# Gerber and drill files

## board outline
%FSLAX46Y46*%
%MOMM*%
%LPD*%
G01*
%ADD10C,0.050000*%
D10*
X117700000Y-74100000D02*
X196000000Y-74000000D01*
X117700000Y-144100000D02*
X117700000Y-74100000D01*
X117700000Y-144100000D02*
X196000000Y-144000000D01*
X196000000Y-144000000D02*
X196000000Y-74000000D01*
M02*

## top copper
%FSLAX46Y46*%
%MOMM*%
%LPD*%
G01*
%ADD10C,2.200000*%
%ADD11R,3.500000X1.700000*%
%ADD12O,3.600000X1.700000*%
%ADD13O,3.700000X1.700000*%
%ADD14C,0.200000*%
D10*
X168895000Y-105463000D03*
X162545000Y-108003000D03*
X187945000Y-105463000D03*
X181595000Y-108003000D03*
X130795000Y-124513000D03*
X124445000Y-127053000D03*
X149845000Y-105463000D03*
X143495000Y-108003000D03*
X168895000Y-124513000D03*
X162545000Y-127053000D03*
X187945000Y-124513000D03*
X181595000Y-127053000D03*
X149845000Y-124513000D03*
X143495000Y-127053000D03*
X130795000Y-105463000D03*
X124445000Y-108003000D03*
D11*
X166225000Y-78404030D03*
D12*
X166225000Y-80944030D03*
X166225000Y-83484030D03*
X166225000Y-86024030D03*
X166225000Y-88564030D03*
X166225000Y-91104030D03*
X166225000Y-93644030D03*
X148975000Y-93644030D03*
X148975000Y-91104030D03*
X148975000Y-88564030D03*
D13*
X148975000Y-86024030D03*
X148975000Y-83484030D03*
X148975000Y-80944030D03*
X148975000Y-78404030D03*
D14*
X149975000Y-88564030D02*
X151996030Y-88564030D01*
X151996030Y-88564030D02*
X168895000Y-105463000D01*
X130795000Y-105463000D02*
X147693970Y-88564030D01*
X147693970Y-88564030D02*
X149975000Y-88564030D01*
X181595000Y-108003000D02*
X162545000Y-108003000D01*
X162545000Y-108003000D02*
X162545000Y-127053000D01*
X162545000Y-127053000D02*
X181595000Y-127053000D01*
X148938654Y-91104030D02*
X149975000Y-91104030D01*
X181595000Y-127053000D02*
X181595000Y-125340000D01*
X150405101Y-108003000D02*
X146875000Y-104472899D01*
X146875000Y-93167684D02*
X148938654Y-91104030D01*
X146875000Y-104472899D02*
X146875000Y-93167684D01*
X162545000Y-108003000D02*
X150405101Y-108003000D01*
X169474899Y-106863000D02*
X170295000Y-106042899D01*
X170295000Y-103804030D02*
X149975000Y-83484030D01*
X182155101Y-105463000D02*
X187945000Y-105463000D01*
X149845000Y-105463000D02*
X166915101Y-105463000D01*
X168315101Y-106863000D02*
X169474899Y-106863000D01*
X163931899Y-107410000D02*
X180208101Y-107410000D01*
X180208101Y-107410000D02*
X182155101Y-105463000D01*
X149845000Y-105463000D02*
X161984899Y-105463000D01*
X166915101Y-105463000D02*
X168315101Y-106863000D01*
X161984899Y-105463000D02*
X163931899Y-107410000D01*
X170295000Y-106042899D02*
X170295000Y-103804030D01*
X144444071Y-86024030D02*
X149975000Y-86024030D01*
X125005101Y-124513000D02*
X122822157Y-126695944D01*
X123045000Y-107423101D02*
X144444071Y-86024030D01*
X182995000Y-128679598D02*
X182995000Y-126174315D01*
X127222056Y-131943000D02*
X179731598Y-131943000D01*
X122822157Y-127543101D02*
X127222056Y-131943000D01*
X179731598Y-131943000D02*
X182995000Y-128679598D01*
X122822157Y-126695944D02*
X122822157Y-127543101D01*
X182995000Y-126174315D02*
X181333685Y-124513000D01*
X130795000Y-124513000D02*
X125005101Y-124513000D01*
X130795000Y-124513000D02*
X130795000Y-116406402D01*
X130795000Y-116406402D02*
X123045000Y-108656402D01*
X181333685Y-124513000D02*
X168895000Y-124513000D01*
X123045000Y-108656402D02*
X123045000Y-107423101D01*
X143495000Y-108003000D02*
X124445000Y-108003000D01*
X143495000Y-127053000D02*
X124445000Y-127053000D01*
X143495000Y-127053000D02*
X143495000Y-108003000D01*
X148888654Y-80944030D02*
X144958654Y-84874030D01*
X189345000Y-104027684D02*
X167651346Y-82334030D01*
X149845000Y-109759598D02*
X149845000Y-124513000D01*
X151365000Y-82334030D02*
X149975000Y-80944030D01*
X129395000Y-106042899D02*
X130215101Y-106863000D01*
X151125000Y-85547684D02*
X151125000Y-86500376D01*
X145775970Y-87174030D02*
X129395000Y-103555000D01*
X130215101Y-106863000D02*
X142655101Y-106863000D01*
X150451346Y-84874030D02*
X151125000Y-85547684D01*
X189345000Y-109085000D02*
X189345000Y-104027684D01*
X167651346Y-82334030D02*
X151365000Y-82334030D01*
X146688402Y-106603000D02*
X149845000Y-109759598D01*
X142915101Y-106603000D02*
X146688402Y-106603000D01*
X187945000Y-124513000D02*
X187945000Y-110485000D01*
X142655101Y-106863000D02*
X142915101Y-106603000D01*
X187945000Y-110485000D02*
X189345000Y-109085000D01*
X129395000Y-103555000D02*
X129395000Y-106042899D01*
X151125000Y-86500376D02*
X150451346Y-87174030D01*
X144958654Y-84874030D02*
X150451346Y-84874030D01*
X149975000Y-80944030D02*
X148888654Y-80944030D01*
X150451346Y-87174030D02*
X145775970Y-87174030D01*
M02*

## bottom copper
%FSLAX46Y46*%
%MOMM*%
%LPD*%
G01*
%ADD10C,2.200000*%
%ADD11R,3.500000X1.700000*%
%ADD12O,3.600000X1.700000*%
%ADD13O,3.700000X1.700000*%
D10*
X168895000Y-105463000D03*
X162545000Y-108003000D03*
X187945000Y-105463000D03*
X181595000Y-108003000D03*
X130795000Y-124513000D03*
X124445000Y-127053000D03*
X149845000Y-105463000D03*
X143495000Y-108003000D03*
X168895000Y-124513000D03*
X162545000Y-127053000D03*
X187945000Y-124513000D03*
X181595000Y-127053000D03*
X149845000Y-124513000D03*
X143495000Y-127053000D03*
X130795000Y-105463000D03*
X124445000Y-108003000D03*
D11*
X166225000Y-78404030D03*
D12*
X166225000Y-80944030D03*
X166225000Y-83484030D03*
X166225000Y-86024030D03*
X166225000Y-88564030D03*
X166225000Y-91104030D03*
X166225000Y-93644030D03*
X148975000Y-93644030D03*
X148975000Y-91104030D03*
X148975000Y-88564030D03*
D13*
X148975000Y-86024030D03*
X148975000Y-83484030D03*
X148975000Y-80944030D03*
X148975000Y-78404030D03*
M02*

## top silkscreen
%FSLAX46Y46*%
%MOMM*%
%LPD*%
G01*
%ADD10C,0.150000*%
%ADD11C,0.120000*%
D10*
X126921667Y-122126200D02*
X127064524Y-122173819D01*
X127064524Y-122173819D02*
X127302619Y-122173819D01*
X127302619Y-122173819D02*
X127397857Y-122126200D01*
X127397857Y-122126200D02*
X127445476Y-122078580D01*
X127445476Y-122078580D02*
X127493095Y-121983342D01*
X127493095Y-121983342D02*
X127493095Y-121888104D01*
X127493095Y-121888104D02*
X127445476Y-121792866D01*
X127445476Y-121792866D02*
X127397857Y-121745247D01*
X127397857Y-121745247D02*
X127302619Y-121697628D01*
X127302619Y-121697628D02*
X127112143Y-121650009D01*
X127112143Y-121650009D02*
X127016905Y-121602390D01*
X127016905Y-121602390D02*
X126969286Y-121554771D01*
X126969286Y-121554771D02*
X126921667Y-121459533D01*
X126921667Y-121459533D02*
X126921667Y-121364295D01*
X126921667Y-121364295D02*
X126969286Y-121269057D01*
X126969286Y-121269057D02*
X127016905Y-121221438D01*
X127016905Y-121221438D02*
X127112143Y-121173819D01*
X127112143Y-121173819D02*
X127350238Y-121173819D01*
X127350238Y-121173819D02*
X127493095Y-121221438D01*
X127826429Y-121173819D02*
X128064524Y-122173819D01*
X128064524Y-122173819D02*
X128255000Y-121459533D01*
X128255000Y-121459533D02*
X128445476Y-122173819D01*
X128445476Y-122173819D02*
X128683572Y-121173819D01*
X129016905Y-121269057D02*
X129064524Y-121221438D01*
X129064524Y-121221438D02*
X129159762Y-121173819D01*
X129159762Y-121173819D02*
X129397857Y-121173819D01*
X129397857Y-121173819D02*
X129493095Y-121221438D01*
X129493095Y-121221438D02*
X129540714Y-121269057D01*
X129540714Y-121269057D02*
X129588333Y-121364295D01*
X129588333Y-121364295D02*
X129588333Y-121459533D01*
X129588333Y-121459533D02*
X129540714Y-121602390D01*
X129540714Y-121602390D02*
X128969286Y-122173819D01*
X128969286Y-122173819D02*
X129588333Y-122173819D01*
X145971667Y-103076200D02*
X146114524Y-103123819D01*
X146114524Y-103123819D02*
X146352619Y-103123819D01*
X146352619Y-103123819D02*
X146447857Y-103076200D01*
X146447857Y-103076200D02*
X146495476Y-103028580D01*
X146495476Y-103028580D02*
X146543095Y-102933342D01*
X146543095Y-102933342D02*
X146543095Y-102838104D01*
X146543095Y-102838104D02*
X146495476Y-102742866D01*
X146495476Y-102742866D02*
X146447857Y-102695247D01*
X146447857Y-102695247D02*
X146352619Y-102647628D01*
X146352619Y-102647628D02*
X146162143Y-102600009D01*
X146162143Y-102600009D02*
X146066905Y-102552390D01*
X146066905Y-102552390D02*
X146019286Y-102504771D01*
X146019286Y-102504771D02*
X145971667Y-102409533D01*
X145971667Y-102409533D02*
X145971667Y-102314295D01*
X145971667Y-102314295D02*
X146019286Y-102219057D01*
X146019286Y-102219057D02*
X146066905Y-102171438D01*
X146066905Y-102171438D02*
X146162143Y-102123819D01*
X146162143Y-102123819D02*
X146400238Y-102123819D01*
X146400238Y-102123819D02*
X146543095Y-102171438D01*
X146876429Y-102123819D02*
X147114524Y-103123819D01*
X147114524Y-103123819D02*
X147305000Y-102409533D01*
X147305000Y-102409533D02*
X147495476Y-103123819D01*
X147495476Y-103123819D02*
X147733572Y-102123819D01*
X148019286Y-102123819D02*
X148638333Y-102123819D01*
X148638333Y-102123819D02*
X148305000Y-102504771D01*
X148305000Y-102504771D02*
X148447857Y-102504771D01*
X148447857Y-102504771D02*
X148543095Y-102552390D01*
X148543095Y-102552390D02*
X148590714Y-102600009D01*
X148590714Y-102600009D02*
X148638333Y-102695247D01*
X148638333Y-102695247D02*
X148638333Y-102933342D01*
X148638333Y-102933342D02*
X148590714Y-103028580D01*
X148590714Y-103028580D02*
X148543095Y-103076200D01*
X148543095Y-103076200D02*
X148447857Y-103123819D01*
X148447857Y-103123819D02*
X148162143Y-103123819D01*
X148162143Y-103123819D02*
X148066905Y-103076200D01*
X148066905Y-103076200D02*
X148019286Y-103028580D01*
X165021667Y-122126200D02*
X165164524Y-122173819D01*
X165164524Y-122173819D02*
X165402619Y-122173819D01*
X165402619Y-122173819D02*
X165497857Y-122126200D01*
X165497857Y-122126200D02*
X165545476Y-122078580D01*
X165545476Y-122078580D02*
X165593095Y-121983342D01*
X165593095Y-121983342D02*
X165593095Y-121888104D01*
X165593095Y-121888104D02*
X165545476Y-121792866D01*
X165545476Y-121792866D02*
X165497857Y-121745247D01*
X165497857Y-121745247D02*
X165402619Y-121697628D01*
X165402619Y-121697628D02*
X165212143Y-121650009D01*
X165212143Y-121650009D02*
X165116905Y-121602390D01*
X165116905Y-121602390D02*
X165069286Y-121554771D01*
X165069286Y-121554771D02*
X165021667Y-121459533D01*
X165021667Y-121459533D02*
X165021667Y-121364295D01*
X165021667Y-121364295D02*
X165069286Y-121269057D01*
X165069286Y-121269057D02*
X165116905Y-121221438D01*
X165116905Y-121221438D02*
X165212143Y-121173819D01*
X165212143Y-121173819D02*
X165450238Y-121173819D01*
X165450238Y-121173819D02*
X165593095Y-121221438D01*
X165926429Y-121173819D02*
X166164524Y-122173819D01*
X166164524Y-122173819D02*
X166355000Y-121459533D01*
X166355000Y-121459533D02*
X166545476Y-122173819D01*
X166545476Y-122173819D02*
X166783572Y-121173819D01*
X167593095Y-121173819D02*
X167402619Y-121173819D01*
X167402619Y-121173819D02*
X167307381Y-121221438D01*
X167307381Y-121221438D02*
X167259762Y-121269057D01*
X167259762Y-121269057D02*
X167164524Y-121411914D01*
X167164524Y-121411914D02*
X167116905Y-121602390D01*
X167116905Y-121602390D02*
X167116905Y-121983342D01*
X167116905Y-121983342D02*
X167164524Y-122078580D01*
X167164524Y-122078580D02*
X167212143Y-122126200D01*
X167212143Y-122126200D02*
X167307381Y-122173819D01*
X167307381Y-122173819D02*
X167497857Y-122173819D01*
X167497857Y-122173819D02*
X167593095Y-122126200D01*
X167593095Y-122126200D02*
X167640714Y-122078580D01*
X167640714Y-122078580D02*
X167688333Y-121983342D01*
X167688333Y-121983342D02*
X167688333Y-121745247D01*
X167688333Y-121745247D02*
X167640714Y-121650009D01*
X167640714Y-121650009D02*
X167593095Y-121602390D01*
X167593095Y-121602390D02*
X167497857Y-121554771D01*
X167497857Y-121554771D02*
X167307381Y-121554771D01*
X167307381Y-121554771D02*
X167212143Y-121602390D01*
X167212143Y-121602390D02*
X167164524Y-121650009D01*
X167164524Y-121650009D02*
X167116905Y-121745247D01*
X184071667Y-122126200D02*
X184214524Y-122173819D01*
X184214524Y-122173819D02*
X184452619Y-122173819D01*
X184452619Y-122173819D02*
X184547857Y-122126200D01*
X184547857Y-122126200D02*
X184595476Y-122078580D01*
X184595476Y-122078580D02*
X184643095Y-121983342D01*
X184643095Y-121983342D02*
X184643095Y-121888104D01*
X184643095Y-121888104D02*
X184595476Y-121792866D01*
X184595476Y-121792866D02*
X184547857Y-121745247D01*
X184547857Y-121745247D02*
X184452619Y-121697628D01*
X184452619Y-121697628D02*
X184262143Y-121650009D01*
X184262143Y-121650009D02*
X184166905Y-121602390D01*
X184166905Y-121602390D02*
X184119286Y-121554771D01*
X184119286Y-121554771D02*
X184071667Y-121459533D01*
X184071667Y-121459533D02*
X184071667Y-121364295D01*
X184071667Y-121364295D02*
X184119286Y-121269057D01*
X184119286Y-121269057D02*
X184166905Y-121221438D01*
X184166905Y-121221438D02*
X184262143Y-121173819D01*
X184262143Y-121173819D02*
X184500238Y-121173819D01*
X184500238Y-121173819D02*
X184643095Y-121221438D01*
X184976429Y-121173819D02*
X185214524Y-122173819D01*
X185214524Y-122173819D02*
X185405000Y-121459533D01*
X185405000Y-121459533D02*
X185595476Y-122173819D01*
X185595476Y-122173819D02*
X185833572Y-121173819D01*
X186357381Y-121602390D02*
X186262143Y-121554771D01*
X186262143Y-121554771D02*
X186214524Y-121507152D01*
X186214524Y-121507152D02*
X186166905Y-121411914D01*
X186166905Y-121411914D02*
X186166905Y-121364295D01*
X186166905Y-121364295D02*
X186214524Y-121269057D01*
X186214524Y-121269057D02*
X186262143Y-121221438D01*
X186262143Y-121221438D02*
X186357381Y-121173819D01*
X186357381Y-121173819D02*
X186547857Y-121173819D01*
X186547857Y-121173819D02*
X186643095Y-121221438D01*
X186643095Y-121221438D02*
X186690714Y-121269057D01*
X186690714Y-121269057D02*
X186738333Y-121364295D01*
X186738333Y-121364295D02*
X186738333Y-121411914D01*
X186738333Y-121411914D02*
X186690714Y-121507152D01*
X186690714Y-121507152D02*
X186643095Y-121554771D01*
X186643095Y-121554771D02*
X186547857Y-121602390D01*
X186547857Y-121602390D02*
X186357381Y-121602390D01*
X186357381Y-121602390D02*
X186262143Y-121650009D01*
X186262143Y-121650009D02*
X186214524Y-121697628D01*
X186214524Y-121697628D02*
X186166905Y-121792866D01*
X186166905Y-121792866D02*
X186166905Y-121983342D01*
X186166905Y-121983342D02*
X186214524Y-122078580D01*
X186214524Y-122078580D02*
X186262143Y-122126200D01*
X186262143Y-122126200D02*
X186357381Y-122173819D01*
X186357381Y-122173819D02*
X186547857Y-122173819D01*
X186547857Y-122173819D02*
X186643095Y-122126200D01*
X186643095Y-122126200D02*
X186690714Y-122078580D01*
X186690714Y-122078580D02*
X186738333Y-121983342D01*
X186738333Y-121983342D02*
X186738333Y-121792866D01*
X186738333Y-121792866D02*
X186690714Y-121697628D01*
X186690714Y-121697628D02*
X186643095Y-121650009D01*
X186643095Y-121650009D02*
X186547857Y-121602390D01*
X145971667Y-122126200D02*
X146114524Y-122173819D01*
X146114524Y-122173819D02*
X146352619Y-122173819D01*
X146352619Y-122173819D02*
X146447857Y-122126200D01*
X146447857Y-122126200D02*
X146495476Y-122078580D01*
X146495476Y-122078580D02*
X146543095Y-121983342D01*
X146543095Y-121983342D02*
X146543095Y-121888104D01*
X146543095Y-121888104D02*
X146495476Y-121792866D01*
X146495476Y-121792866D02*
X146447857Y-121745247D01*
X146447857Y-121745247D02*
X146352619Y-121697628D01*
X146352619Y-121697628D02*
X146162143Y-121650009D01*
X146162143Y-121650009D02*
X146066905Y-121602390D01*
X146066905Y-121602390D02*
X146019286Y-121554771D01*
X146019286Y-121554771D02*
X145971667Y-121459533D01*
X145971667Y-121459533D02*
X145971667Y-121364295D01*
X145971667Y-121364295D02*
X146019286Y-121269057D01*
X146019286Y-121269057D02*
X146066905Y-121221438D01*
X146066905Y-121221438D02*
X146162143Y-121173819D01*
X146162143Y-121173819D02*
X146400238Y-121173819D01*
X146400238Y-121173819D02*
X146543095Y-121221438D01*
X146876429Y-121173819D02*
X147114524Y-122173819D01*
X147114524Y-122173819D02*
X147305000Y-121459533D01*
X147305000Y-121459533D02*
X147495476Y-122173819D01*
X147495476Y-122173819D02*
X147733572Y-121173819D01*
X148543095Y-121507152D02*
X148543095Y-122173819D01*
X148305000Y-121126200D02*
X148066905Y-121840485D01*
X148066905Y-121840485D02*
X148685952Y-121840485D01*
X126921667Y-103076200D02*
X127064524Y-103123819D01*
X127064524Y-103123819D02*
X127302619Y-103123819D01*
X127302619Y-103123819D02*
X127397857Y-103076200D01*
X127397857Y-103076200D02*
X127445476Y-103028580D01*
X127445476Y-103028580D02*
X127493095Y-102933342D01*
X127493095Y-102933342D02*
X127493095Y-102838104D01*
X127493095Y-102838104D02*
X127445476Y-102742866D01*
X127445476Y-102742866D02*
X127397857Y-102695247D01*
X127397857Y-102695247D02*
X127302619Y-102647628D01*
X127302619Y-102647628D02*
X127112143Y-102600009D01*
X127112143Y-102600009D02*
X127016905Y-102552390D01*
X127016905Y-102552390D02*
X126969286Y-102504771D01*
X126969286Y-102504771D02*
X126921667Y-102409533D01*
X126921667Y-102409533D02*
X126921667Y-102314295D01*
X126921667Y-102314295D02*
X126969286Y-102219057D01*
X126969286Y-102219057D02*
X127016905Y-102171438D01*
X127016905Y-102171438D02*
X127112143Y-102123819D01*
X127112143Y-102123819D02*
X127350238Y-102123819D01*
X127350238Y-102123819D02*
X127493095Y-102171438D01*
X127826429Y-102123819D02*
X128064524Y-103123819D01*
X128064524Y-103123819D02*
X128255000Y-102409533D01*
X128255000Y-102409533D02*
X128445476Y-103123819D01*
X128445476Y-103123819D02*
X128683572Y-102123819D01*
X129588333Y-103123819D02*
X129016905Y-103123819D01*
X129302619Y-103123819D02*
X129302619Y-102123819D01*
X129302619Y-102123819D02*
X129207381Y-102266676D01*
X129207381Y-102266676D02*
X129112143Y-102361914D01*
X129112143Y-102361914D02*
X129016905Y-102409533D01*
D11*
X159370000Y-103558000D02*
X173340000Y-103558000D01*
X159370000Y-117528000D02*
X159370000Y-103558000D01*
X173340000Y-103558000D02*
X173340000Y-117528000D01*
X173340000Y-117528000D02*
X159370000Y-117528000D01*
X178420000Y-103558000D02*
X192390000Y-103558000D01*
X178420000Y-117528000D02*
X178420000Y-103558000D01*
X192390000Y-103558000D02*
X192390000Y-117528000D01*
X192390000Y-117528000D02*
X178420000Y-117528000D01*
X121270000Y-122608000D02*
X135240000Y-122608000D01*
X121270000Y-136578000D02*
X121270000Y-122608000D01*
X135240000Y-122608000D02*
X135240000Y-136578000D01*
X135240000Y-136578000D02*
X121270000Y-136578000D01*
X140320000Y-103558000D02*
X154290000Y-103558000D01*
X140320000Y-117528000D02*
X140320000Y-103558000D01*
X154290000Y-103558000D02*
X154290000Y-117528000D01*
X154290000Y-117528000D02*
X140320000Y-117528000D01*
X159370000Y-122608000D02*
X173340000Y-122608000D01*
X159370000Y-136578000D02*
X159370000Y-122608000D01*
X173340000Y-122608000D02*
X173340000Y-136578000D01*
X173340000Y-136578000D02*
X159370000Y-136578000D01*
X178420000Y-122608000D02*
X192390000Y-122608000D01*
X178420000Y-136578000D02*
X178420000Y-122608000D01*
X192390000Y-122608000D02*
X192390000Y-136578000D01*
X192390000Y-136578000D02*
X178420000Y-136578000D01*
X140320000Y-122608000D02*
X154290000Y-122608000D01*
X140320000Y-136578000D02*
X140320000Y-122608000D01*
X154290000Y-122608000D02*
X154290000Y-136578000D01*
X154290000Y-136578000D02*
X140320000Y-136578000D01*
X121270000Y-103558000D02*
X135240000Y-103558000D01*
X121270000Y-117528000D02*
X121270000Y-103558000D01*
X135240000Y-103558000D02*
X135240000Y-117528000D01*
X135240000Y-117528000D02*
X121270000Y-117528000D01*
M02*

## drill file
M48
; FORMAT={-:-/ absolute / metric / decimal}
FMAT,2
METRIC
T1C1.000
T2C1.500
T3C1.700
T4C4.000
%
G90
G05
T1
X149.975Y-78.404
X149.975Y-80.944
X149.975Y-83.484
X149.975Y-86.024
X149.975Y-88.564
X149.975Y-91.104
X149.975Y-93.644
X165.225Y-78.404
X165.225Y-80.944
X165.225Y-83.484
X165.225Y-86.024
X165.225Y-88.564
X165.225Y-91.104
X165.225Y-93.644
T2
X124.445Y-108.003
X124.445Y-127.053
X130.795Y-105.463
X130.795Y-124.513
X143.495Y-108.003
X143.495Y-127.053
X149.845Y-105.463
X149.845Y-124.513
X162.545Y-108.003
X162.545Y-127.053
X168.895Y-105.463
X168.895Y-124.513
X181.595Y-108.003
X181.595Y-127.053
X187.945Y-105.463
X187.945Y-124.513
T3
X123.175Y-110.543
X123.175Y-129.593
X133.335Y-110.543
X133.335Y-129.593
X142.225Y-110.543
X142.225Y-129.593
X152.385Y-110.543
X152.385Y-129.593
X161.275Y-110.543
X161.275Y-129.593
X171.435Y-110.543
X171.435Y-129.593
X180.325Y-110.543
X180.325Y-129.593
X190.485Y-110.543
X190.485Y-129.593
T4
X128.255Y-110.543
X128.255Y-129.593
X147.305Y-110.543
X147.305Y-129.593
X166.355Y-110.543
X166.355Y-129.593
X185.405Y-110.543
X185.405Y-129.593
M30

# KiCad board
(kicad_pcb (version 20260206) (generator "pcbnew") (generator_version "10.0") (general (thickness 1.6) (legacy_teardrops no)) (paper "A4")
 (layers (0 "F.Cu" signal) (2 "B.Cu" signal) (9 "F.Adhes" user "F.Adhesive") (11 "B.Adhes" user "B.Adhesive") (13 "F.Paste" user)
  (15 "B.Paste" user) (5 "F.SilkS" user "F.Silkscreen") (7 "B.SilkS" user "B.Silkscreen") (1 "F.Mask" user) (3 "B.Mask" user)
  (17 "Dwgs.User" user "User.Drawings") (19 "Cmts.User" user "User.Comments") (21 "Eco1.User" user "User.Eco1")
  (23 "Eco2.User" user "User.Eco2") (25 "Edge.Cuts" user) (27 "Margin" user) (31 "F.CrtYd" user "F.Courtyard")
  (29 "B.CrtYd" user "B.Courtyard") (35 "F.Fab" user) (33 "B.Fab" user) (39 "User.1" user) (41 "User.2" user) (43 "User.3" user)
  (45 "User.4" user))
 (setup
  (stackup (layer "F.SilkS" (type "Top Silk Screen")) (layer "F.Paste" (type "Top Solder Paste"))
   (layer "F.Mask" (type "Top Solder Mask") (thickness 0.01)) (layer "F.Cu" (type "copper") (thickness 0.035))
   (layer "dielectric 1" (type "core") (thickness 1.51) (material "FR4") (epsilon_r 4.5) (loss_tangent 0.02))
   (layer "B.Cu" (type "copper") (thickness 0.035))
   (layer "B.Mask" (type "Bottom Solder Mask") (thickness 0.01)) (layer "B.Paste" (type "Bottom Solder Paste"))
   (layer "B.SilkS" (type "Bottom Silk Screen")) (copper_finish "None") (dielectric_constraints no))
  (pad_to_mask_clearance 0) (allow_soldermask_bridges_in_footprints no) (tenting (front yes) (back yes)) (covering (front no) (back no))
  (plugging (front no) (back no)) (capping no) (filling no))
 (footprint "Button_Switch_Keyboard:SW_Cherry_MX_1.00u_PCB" (layer "F.Cu") (at 168.895 105.463)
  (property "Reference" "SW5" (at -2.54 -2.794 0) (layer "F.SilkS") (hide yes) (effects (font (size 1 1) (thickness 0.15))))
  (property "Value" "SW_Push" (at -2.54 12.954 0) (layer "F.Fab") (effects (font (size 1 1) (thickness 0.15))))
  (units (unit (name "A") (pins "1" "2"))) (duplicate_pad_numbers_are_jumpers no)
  (fp_line (start -9.525 -1.905) (end 4.445 -1.905) (stroke (width 0.12) (type solid)) (layer "F.SilkS"))
  (fp_line (start -9.525 12.065) (end -9.525 -1.905) (stroke (width 0.12) (type solid)) (layer "F.SilkS"))
  (fp_line (start 4.445 -1.905) (end 4.445 12.065) (stroke (width 0.12) (type solid)) (layer "F.SilkS"))
  (fp_line (start 4.445 12.065) (end -9.525 12.065) (stroke (width 0.12) (type solid)) (layer "F.SilkS"))
  (pad "" np_thru_hole circle (at -7.62 5.08) (size 1.7 1.7) (drill 1.7) (layers "*.Cu" "*.Mask"))
  (pad "" np_thru_hole circle (at -2.54 5.08) (size 4 4) (drill 4) (layers "*.Cu" "*.Mask"))
  (pad "" np_thru_hole circle (at 2.54 5.08) (size 1.7 1.7) (drill 1.7) (layers "*.Cu" "*.Mask"))
  (pad "1" thru_hole circle (at 0 0) (size 2.2 2.2) (drill 1.5) (layers "*.Cu" "*.Mask") (remove_unused_layers no)
   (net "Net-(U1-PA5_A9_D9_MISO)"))
  (pad "2" thru_hole circle (at -6.35 2.54) (size 2.2 2.2) (drill 1.5) (layers "*.Cu" "*.Mask") (remove_unused_layers no)
   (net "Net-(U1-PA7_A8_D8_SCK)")))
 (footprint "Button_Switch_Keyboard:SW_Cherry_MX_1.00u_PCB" (layer "F.Cu") (at 187.945 105.463)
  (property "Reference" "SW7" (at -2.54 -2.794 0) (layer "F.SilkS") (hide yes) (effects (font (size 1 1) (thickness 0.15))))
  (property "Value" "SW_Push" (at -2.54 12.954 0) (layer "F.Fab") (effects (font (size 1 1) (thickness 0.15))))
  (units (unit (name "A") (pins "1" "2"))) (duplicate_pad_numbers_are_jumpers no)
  (fp_line (start -9.525 -1.905) (end 4.445 -1.905) (stroke (width 0.12) (type solid)) (layer "F.SilkS"))
  (fp_line (start -9.525 12.065) (end -9.525 -1.905) (stroke (width 0.12) (type solid)) (layer "F.SilkS"))
  (fp_line (start 4.445 -1.905) (end 4.445 12.065) (stroke (width 0.12) (type solid)) (layer "F.SilkS"))
  (fp_line (start 4.445 12.065) (end -9.525 12.065) (stroke (width 0.12) (type solid)) (layer "F.SilkS"))
  (pad "" np_thru_hole circle (at -7.62 5.08) (size 1.7 1.7) (drill 1.7) (layers "*.Cu" "*.Mask"))
  (pad "" np_thru_hole circle (at -2.54 5.08) (size 4 4) (drill 4) (layers "*.Cu" "*.Mask"))
  (pad "" np_thru_hole circle (at 2.54 5.08) (size 1.7 1.7) (drill 1.7) (layers "*.Cu" "*.Mask"))
  (pad "1" thru_hole circle (at 0 0) (size 2.2 2.2) (drill 1.5) (layers "*.Cu" "*.Mask") (remove_unused_layers no) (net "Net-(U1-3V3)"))
  (pad "2" thru_hole circle (at -6.35 2.54) (size 2.2 2.2) (drill 1.5) (layers "*.Cu" "*.Mask") (remove_unused_layers no)
   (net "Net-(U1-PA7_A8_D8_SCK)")))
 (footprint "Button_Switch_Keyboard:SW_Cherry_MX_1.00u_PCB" (layer "F.Cu") (at 130.795 124.513)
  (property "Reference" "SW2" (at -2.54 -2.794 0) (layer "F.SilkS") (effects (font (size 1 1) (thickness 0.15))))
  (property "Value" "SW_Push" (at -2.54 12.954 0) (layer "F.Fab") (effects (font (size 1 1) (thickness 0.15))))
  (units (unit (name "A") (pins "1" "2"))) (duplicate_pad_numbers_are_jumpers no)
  (fp_line (start -9.525 -1.905) (end 4.445 -1.905) (stroke (width 0.12) (type solid)) (layer "F.SilkS"))
  (fp_line (start -9.525 12.065) (end -9.525 -1.905) (stroke (width 0.12) (type solid)) (layer "F.SilkS"))
  (fp_line (start 4.445 -1.905) (end 4.445 12.065) (stroke (width 0.12) (type solid)) (layer "F.SilkS"))
  (fp_line (start 4.445 12.065) (end -9.525 12.065) (stroke (width 0.12) (type solid)) (layer "F.SilkS"))
  (pad "" np_thru_hole circle (at -7.62 5.08) (size 1.7 1.7) (drill 1.7) (layers "*.Cu" "*.Mask"))
  (pad "" np_thru_hole circle (at -2.54 5.08) (size 4 4) (drill 4) (layers "*.Cu" "*.Mask"))
  (pad "" np_thru_hole circle (at 2.54 5.08) (size 1.7 1.7) (drill 1.7) (layers "*.Cu" "*.Mask"))
  (pad "1" thru_hole circle (at 0 0) (size 2.2 2.2) (drill 1.5) (layers "*.Cu" "*.Mask") (remove_unused_layers no)
   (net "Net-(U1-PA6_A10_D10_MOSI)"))
  (pad "2" thru_hole circle (at -6.35 2.54) (size 2.2 2.2) (drill 1.5) (layers "*.Cu" "*.Mask") (remove_unused_layers no)
   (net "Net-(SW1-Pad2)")))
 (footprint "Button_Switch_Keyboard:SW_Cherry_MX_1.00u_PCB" (layer "F.Cu") (at 149.845 105.463)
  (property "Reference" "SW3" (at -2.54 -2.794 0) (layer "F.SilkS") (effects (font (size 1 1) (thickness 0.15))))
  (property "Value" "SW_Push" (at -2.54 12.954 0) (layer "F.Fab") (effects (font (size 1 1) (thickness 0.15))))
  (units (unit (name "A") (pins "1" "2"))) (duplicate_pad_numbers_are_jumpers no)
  (fp_line (start -9.525 -1.905) (end 4.445 -1.905) (stroke (width 0.12) (type solid)) (layer "F.SilkS"))
  (fp_line (start -9.525 12.065) (end -9.525 -1.905) (stroke (width 0.12) (type solid)) (layer "F.SilkS"))
  (fp_line (start 4.445 -1.905) (end 4.445 12.065) (stroke (width 0.12) (type solid)) (layer "F.SilkS"))
  (fp_line (start 4.445 12.065) (end -9.525 12.065) (stroke (width 0.12) (type solid)) (layer "F.SilkS"))
  (pad "" np_thru_hole circle (at -7.62 5.08) (size 1.7 1.7) (drill 1.7) (layers "*.Cu" "*.Mask"))
  (pad "" np_thru_hole circle (at -2.54 5.08) (size 4 4) (drill 4) (layers "*.Cu" "*.Mask"))
  (pad "" np_thru_hole circle (at 2.54 5.08) (size 1.7 1.7) (drill 1.7) (layers "*.Cu" "*.Mask"))
  (pad "1" thru_hole circle (at 0 0) (size 2.2 2.2) (drill 1.5) (layers "*.Cu" "*.Mask") (remove_unused_layers no) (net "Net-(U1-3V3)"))
  (pad "2" thru_hole circle (at -6.35 2.54) (size 2.2 2.2) (drill 1.5) (layers "*.Cu" "*.Mask") (remove_unused_layers no)
   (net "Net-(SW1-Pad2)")))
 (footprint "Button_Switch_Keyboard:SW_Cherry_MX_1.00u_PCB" (layer "F.Cu") (at 168.895 124.513)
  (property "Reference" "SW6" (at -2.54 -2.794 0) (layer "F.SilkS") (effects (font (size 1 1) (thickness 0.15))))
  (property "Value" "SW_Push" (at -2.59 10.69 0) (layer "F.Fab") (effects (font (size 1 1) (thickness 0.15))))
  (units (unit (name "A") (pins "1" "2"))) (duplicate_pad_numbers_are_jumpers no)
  (fp_line (start -9.525 -1.905) (end 4.445 -1.905) (stroke (width 0.12) (type solid)) (layer "F.SilkS"))
  (fp_line (start -9.525 12.065) (end -9.525 -1.905) (stroke (width 0.12) (type solid)) (layer "F.SilkS"))
  (fp_line (start 4.445 -1.905) (end 4.445 12.065) (stroke (width 0.12) (type solid)) (layer "F.SilkS"))
  (fp_line (start 4.445 12.065) (end -9.525 12.065) (stroke (width 0.12) (type solid)) (layer "F.SilkS"))
  (pad "" np_thru_hole circle (at -7.62 5.08) (size 1.7 1.7) (drill 1.7) (layers "*.Cu" "*.Mask"))
  (pad "" np_thru_hole circle (at -2.54 5.08) (size 4 4) (drill 4) (layers "*.Cu" "*.Mask"))
  (pad "" np_thru_hole circle (at 2.54 5.08) (size 1.7 1.7) (drill 1.7) (layers "*.Cu" "*.Mask"))
  (pad "1" thru_hole circle (at 0 0) (size 2.2 2.2) (drill 1.5) (layers "*.Cu" "*.Mask") (remove_unused_layers no)
   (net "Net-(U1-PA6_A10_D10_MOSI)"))
  (pad "2" thru_hole circle (at -6.35 2.54) (size 2.2 2.2) (drill 1.5) (layers "*.Cu" "*.Mask") (remove_unused_layers no)
   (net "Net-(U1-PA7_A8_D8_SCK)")))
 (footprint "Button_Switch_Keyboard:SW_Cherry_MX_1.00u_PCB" (layer "F.Cu") (at 187.945 124.513)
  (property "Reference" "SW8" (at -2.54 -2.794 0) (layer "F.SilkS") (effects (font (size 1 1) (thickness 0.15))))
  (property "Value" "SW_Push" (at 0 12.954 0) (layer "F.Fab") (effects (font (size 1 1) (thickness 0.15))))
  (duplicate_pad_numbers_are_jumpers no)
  (fp_line (start -9.525 -1.905) (end 4.445 -1.905) (stroke (width 0.12) (type solid)) (layer "F.SilkS"))
  (fp_line (start -9.525 12.065) (end -9.525 -1.905) (stroke (width 0.12) (type solid)) (layer "F.SilkS"))
  (fp_line (start 4.445 -1.905) (end 4.445 12.065) (stroke (width 0.12) (type solid)) (layer "F.SilkS"))
  (fp_line (start 4.445 12.065) (end -9.525 12.065) (stroke (width 0.12) (type solid)) (layer "F.SilkS"))
  (pad "" np_thru_hole circle (at -7.62 5.08) (size 1.7 1.7) (drill 1.7) (layers "*.Cu" "*.Mask"))
  (pad "" np_thru_hole circle (at -2.54 5.08) (size 4 4) (drill 4) (layers "*.Cu" "*.Mask"))
  (pad "" np_thru_hole circle (at 2.54 5.08) (size 1.7 1.7) (drill 1.7) (layers "*.Cu" "*.Mask"))
  (pad "1" thru_hole circle (at 0 0) (size 2.2 2.2) (drill 1.5) (layers "*.Cu" "*.Mask") (remove_unused_layers no) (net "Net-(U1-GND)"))
  (pad "2" thru_hole circle (at -6.35 2.54) (size 2.2 2.2) (drill 1.5) (layers "*.Cu" "*.Mask") (remove_unused_layers no)
   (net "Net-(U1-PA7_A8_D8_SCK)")))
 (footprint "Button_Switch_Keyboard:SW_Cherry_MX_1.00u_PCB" (layer "F.Cu") (at 149.845 124.513)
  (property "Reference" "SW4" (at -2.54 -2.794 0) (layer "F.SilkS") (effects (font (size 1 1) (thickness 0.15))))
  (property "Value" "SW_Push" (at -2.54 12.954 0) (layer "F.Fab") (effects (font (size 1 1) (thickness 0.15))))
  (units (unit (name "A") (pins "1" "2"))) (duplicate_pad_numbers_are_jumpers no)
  (fp_line (start -9.525 -1.905) (end 4.445 -1.905) (stroke (width 0.12) (type solid)) (layer "F.SilkS"))
  (fp_line (start -9.525 12.065) (end -9.525 -1.905) (stroke (width 0.12) (type solid)) (layer "F.SilkS"))
  (fp_line (start 4.445 -1.905) (end 4.445 12.065) (stroke (width 0.12) (type solid)) (layer "F.SilkS"))
  (fp_line (start 4.445 12.065) (end -9.525 12.065) (stroke (width 0.12) (type solid)) (layer "F.SilkS"))
  (pad "" np_thru_hole circle (at -7.62 5.08) (size 1.7 1.7) (drill 1.7) (layers "*.Cu" "*.Mask"))
  (pad "" np_thru_hole circle (at -2.54 5.08) (size 4 4) (drill 4) (layers "*.Cu" "*.Mask"))
  (pad "" np_thru_hole circle (at 2.54 5.08) (size 1.7 1.7) (drill 1.7) (layers "*.Cu" "*.Mask"))
  (pad "1" thru_hole circle (at 0 0) (size 2.2 2.2) (drill 1.5) (layers "*.Cu" "*.Mask") (remove_unused_layers no) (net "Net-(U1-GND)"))
  (pad "2" thru_hole circle (at -6.35 2.54) (size 2.2 2.2) (drill 1.5) (layers "*.Cu" "*.Mask") (remove_unused_layers no)
   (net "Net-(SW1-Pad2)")))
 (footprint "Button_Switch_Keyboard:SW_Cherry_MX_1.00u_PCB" (layer "F.Cu") (at 130.795 105.463)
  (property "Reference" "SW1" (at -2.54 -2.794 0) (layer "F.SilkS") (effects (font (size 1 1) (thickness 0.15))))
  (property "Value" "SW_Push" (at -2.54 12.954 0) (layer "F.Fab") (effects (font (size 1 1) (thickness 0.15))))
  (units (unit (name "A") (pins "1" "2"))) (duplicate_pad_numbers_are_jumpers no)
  (fp_line (start -9.525 -1.905) (end 4.445 -1.905) (stroke (width 0.12) (type solid)) (layer "F.SilkS"))
  (fp_line (start -9.525 12.065) (end -9.525 -1.905) (stroke (width 0.12) (type solid)) (layer "F.SilkS"))
  (fp_line (start 4.445 -1.905) (end 4.445 12.065) (stroke (width 0.12) (type solid)) (layer "F.SilkS"))
  (fp_line (start 4.445 12.065) (end -9.525 12.065) (stroke (width 0.12) (type solid)) (layer "F.SilkS"))
  (pad "" np_thru_hole circle (at -7.62 5.08) (size 1.7 1.7) (drill 1.7) (layers "*.Cu" "*.Mask"))
  (pad "" np_thru_hole circle (at -2.54 5.08) (size 4 4) (drill 4) (layers "*.Cu" "*.Mask"))
  (pad "" np_thru_hole circle (at 2.54 5.08) (size 1.7 1.7) (drill 1.7) (layers "*.Cu" "*.Mask"))
  (pad "1" thru_hole circle (at 0 0) (size 2.2 2.2) (drill 1.5) (layers "*.Cu" "*.Mask") (remove_unused_layers no)
   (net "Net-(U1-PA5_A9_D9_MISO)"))
  (pad "2" thru_hole circle (at -6.35 2.54) (size 2.2 2.2) (drill 1.5) (layers "*.Cu" "*.Mask") (remove_unused_layers no)
   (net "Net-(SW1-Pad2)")))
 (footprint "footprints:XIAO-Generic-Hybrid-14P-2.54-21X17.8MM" (layer "B.Cu") (at 157.6 86.02403 180)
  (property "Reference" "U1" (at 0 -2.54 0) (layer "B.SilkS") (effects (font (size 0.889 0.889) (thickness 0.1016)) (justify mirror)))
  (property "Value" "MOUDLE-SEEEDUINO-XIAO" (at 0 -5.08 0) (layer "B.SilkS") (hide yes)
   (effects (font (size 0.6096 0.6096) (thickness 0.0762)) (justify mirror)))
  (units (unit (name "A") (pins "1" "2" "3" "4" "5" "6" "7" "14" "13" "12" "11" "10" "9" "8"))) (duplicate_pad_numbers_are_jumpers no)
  (pad "1" thru_hole rect (at -7.625 7.62 180) (size 3.5 1.7) (drill 1 (offset -1 0)) (layers "*.Cu" "*.Mask") (remove_unused_layers no)
   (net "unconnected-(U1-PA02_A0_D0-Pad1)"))
  (pad "2" thru_hole oval (at -7.625 5.08 180) (size 3.6 1.7) (drill 1 (offset -1 0)) (layers "*.Cu" "*.Mask") (remove_unused_layers no)
   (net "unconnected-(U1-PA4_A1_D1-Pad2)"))
  (pad "3" thru_hole oval (at -7.625 2.54 180) (size 3.6 1.7) (drill 1 (offset -1 0)) (layers "*.Cu" "*.Mask") (remove_unused_layers no)
   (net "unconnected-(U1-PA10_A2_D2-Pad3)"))
  (pad "4" thru_hole oval (at -7.625 0 180) (size 3.6 1.7) (drill 1 (offset -1 0)) (layers "*.Cu" "*.Mask") (remove_unused_layers no)
   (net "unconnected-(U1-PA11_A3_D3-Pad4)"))
  (pad "5" thru_hole oval (at -7.625 -2.54 180) (size 3.6 1.7) (drill 1 (offset -1 0)) (layers "*.Cu" "*.Mask") (remove_unused_layers no)
   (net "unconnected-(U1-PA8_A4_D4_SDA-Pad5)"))
  (pad "6" thru_hole oval (at -7.625 -5.08) (size 3.6 1.7) (drill 1 (offset 1 0)) (layers "*.Cu" "*.Mask") (remove_unused_layers no)
   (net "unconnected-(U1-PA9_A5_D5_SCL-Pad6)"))
  (pad "7" thru_hole oval (at -7.625 -7.62 180) (size 3.6 1.7) (drill 1 (offset -1 0)) (layers "*.Cu" "*.Mask") (remove_unused_layers no)
   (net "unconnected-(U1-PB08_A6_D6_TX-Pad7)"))
  (pad "8" thru_hole oval (at 7.625 -7.62 180) (size 3.6 1.7) (drill 1 (offset 1 0)) (layers "*.Cu" "*.Mask") (remove_unused_layers no)
   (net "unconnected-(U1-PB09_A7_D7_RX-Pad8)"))
  (pad "9" thru_hole oval (at 7.625 -5.08 180) (size 3.6 1.7) (drill 1 (offset 1 0)) (layers "*.Cu" "*.Mask") (remove_unused_layers no)
   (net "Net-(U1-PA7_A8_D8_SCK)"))
  (pad "10" thru_hole oval (at 7.625 -2.54 180) (size 3.6 1.7) (drill 1 (offset 1 0)) (layers "*.Cu" "*.Mask") (remove_unused_layers no)
   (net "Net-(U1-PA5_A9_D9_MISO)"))
  (pad "11" thru_hole oval (at 7.625 0 180) (size 3.7 1.7) (drill 1 (offset 1 0)) (layers "*.Cu" "*.Mask") (remove_unused_layers no)
   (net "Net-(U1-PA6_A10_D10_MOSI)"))
  (pad "12" thru_hole oval (at 7.625 2.54 180) (size 3.7 1.7) (drill 1 (offset 1 0)) (layers "*.Cu" "*.Mask") (remove_unused_layers no)
   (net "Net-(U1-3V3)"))
  (pad "13" thru_hole oval (at 7.625 5.08 180) (size 3.7 1.7) (drill 1 (offset 1 0)) (layers "*.Cu" "*.Mask") (remove_unused_layers no)
   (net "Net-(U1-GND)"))
  (pad "14" thru_hole oval (at 7.625 7.62 180) (size 3.7 1.7) (drill 1 (offset 1 0)) (layers "*.Cu" "*.Mask") (remove_unused_layers no)
   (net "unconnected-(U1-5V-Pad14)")))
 (gr_line (start 117.7 74.1) (end 196 74) (stroke (width 0.05) (type default)) (layer "Edge.Cuts"))
 (gr_line (start 117.7 144.1) (end 117.7 74.1) (stroke (width 0.05) (type default)) (layer "Edge.Cuts"))
 (gr_line (start 117.7 144.1) (end 196 144) (stroke (width 0.05) (type default)) (layer "Edge.Cuts"))
 (gr_line (start 196 144) (end 196 74) (stroke (width 0.05) (type default)) (layer "Edge.Cuts"))
 (segment (start 149.975 88.56403) (end 151.99603 88.56403) (width 0.2) (layer "F.Cu") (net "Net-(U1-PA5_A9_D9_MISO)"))
 (segment (start 151.99603 88.56403) (end 168.895 105.463) (width 0.2) (layer "F.Cu") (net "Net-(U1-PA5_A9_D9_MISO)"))
 (segment (start 130.795 105.463) (end 147.69397 88.56403) (width 0.2) (layer "F.Cu") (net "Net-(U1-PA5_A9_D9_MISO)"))
 (segment (start 147.69397 88.56403) (end 149.975 88.56403) (width 0.2) (layer "F.Cu") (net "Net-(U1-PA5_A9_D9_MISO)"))
 (segment (start 181.595 108.003) (end 162.545 108.003) (width 0.2) (layer "F.Cu") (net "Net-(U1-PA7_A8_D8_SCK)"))
 (segment (start 162.545 108.003) (end 162.545 127.053) (width 0.2) (layer "F.Cu") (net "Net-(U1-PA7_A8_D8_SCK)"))
 (segment (start 162.545 127.053) (end 181.595 127.053) (width 0.2) (layer "F.Cu") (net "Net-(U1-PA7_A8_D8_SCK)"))
 (segment (start 148.938654 91.10403) (end 149.975 91.10403) (width 0.2) (layer "F.Cu") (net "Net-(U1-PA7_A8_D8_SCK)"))
 (segment (start 181.595 127.053) (end 181.595 125.34) (width 0.2) (layer "F.Cu") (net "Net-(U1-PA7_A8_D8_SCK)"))
 (segment (start 150.405101 108.003) (end 146.875 104.472899) (width 0.2) (layer "F.Cu") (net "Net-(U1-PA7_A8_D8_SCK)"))
 (segment (start 146.875 93.167684) (end 148.938654 91.10403) (width 0.2) (layer "F.Cu") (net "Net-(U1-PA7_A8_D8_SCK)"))
 (segment (start 146.875 104.472899) (end 146.875 93.167684) (width 0.2) (layer "F.Cu") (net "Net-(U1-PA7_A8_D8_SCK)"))
 (segment (start 162.545 108.003) (end 150.405101 108.003) (width 0.2) (layer "F.Cu") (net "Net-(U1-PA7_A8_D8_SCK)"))
 (segment (start 169.474899 106.863) (end 170.295 106.042899) (width 0.2) (layer "F.Cu") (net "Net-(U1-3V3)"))
 (segment (start 170.295 103.80403) (end 149.975 83.48403) (width 0.2) (layer "F.Cu") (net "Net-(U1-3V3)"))
 (segment (start 182.155101 105.463) (end 187.945 105.463) (width 0.2) (layer "F.Cu") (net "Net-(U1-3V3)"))
 (segment (start 149.845 105.463) (end 166.915101 105.463) (width 0.2) (layer "F.Cu") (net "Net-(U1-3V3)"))
 (segment (start 168.315101 106.863) (end 169.474899 106.863) (width 0.2) (layer "F.Cu") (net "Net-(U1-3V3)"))
 (segment (start 163.931899 107.41) (end 180.208101 107.41) (width 0.2) (layer "F.Cu") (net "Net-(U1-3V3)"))
 (segment (start 180.208101 107.41) (end 182.155101 105.463) (width 0.2) (layer "F.Cu") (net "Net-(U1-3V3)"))
 (segment (start 149.845 105.463) (end 161.984899 105.463) (width 0.2) (layer "F.Cu") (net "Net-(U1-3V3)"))
 (segment (start 166.915101 105.463) (end 168.315101 106.863) (width 0.2) (layer "F.Cu") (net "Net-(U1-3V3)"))
 (segment (start 161.984899 105.463) (end 163.931899 107.41) (width 0.2) (layer "F.Cu") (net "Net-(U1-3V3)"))
 (segment (start 170.295 106.042899) (end 170.295 103.80403) (width 0.2) (layer "F.Cu") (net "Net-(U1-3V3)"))
 (segment (start 144.444071 86.02403) (end 149.975 86.02403) (width 0.2) (layer "F.Cu") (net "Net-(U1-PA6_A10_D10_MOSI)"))
 (segment (start 125.005101 124.513) (end 122.822157 126.695944) (width 0.2) (layer "F.Cu") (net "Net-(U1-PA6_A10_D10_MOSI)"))
 (segment (start 123.045 107.423101) (end 144.444071 86.02403) (width 0.2) (layer "F.Cu") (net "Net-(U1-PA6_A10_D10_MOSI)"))
 (segment (start 182.995 128.679598) (end 182.995 126.174315) (width 0.2) (layer "F.Cu") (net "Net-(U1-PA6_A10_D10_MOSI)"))
 (segment (start 127.222056 131.943) (end 179.731598 131.943) (width 0.2) (layer "F.Cu") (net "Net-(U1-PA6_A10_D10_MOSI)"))
 (segment (start 122.822157 127.543101) (end 127.222056 131.943) (width 0.2) (layer "F.Cu") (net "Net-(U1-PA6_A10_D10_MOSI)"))
 (segment (start 179.731598 131.943) (end 182.995 128.679598) (width 0.2) (layer "F.Cu") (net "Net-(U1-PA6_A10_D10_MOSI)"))
 (segment (start 122.822157 126.695944) (end 122.822157 127.543101) (width 0.2) (layer "F.Cu") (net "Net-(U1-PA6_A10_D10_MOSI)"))
 (segment (start 182.995 126.174315) (end 181.333685 124.513) (width 0.2) (layer "F.Cu") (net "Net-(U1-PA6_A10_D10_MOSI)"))
 (segment (start 130.795 124.513) (end 125.005101 124.513) (width 0.2) (layer "F.Cu") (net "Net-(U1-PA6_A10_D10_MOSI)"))
 (segment (start 130.795 124.513) (end 130.795 116.406402) (width 0.2) (layer "F.Cu") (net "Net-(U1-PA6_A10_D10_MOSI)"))
 (segment (start 130.795 116.406402) (end 123.045 108.656402) (width 0.2) (layer "F.Cu") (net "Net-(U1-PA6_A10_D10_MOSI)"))
 (segment (start 181.333685 124.513) (end 168.895 124.513) (width 0.2) (layer "F.Cu") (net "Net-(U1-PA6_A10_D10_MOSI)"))
 (segment (start 123.045 108.656402) (end 123.045 107.423101) (width 0.2) (layer "F.Cu") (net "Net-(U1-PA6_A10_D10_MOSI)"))
 (segment (start 143.495 108.003) (end 124.445 108.003) (width 0.2) (layer "F.Cu") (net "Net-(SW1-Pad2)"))
 (segment (start 143.495 127.053) (end 124.445 127.053) (width 0.2) (layer "F.Cu") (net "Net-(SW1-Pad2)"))
 (segment (start 143.495 127.053) (end 143.495 108.003) (width 0.2) (layer "F.Cu") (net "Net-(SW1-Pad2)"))
 (segment (start 148.888654 80.94403) (end 144.958654 84.87403) (width 0.2) (layer "F.Cu") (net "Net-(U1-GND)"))
 (segment (start 189.345 104.027684) (end 167.651346 82.33403) (width 0.2) (layer "F.Cu") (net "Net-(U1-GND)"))
 (segment (start 149.845 109.759598) (end 149.845 124.513) (width 0.2) (layer "F.Cu") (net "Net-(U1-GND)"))
 (segment (start 151.365 82.33403) (end 149.975 80.94403) (width 0.2) (layer "F.Cu") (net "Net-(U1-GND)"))
 (segment (start 129.395 106.042899) (end 130.215101 106.863) (width 0.2) (layer "F.Cu") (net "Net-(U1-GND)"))
 (segment (start 151.125 85.547684) (end 151.125 86.500376) (width 0.2) (layer "F.Cu") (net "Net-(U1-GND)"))
 (segment (start 145.77597 87.17403) (end 129.395 103.555) (width 0.2) (layer "F.Cu") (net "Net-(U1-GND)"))
 (segment (start 130.215101 106.863) (end 142.655101 106.863) (width 0.2) (layer "F.Cu") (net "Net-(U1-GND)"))
 (segment (start 150.451346 84.87403) (end 151.125 85.547684) (width 0.2) (layer "F.Cu") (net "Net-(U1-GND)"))
 (segment (start 189.345 109.085) (end 189.345 104.027684) (width 0.2) (layer "F.Cu") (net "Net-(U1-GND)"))
 (segment (start 167.651346 82.33403) (end 151.365 82.33403) (width 0.2) (layer "F.Cu") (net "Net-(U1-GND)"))
 (segment (start 146.688402 106.603) (end 149.845 109.759598) (width 0.2) (layer "F.Cu") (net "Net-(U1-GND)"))
 (segment (start 142.915101 106.603) (end 146.688402 106.603) (width 0.2) (layer "F.Cu") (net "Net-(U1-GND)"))
 (segment (start 187.945 124.513) (end 187.945 110.485) (width 0.2) (layer "F.Cu") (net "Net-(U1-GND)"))
 (segment (start 142.655101 106.863) (end 142.915101 106.603) (width 0.2) (layer "F.Cu") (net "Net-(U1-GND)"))
 (segment (start 187.945 110.485) (end 189.345 109.085) (width 0.2) (layer "F.Cu") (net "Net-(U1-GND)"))
 (segment (start 129.395 103.555) (end 129.395 106.042899) (width 0.2) (layer "F.Cu") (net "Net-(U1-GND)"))
 (segment (start 151.125 86.500376) (end 150.451346 87.17403) (width 0.2) (layer "F.Cu") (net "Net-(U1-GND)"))
 (segment (start 144.958654 84.87403) (end 150.451346 84.87403) (width 0.2) (layer "F.Cu") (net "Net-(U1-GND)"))
 (segment (start 149.975 80.94403) (end 148.888654 80.94403) (width 0.2) (layer "F.Cu") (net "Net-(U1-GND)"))
 (segment (start 150.451346 87.17403) (end 145.77597 87.17403) (width 0.2) (layer "F.Cu") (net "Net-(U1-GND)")))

